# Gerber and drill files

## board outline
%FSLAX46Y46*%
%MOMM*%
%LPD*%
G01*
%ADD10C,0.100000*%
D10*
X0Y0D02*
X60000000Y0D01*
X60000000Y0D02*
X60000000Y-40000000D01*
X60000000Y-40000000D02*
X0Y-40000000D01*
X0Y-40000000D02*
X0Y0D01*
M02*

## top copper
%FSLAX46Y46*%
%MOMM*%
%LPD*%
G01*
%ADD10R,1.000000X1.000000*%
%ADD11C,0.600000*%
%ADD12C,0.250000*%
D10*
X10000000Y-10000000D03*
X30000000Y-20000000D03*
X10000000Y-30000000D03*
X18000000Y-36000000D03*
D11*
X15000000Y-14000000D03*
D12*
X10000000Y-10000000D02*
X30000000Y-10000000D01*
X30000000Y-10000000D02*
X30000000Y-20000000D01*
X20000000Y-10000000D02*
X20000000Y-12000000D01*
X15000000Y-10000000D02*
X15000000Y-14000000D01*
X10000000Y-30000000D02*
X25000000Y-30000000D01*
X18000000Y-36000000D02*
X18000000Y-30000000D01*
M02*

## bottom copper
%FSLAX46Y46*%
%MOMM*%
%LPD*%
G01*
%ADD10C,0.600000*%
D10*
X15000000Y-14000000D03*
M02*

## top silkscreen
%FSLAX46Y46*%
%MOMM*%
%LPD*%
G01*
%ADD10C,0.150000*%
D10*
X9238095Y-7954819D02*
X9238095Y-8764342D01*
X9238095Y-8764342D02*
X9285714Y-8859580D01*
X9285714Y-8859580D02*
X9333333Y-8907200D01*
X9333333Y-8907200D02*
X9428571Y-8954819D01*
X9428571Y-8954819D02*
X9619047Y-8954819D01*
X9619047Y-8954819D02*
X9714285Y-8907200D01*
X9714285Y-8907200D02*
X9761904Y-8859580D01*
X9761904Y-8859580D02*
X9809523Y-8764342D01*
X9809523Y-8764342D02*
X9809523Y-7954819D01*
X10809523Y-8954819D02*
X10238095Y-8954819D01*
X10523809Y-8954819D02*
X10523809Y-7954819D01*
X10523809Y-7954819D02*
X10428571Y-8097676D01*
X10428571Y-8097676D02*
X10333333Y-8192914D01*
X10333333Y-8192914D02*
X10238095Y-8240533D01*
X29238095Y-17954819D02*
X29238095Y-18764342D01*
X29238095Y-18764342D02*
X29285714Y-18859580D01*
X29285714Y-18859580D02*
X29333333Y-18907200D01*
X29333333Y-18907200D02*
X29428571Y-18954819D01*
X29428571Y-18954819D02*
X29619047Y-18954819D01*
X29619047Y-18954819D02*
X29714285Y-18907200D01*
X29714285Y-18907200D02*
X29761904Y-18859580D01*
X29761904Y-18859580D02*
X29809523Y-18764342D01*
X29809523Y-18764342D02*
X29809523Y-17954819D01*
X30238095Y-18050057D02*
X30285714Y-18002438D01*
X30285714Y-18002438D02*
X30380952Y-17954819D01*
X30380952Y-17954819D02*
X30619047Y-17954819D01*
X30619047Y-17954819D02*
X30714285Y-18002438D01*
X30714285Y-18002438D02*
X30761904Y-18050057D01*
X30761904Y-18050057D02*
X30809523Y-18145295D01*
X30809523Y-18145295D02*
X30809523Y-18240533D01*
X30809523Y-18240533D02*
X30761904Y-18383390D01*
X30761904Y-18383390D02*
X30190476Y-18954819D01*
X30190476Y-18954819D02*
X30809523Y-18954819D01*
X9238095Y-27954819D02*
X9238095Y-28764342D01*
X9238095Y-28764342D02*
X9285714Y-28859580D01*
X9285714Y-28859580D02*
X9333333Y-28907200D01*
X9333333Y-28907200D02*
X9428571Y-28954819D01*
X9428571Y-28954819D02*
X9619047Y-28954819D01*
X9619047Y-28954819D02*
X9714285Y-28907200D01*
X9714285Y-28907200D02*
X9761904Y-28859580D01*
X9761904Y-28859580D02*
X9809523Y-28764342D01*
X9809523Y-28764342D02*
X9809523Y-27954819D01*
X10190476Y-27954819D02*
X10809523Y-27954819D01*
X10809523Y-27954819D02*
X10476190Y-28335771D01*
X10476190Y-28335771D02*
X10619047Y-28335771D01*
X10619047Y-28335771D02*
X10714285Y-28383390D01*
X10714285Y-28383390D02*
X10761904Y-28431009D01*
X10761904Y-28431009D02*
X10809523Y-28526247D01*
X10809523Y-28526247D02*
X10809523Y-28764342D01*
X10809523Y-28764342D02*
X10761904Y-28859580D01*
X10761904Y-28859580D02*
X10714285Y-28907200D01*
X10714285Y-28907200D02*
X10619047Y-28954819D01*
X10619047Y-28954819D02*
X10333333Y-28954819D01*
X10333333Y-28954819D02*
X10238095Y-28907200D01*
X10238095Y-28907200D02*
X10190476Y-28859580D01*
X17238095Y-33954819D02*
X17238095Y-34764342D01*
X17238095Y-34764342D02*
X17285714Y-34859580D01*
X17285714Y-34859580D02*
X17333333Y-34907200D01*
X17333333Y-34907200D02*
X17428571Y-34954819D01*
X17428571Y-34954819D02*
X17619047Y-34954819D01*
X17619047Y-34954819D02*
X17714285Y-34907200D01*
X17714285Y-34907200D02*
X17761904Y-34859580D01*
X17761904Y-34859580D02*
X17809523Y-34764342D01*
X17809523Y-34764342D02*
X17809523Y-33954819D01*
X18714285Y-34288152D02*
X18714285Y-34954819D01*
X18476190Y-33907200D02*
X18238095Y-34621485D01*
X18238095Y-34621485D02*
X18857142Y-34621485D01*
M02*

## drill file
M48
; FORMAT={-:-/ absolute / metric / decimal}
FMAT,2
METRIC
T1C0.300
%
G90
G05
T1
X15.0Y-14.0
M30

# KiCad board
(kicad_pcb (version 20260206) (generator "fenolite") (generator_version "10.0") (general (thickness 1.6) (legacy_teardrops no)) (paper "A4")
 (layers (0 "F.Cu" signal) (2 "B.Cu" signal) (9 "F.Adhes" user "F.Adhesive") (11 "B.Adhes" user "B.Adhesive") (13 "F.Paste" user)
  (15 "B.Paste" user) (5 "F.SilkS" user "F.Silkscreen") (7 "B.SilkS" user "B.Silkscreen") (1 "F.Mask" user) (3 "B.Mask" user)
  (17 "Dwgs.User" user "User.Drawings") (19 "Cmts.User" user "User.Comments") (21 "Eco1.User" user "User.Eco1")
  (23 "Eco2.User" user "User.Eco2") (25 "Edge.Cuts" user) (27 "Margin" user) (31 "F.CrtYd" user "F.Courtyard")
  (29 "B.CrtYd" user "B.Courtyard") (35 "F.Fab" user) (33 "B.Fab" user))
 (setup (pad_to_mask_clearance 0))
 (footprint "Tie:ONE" (layer "F.Cu") (at 10 10)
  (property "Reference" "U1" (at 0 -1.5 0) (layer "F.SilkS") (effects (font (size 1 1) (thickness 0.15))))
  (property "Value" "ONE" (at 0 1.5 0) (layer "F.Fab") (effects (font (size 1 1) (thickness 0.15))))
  (pad "1" smd rect (at 0 0) (size 1 1) (layers "F.Cu" "F.Paste" "F.Mask") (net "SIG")))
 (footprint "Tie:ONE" (layer "F.Cu") (at 30 20)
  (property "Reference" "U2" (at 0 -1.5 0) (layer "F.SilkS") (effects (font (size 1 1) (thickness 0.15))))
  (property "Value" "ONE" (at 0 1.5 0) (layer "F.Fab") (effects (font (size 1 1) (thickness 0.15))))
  (pad "1" smd rect (at 0 0) (size 1 1) (layers "F.Cu" "F.Paste" "F.Mask") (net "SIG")))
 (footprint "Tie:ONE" (layer "F.Cu") (at 10 30)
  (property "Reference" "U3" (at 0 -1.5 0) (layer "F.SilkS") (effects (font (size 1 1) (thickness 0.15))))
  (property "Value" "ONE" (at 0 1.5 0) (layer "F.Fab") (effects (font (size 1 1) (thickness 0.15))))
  (pad "1" smd rect (at 0 0) (size 1 1) (layers "F.Cu" "F.Paste" "F.Mask") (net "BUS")))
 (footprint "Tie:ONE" (layer "F.Cu") (at 18 36)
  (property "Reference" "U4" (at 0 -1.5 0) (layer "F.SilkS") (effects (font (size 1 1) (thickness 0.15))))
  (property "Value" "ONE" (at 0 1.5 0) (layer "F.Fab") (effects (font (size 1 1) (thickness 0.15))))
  (pad "1" smd rect (at 0 0) (size 1 1) (layers "F.Cu" "F.Paste" "F.Mask") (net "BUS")))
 (gr_line (start 0 0) (end 60 0) (stroke (width 0.1) (type solid)) (layer "Edge.Cuts"))
 (gr_line (start 60 0) (end 60 40) (stroke (width 0.1) (type solid)) (layer "Edge.Cuts"))
 (gr_line (start 60 40) (end 0 40) (stroke (width 0.1) (type solid)) (layer "Edge.Cuts"))
 (gr_line (start 0 40) (end 0 0) (stroke (width 0.1) (type solid)) (layer "Edge.Cuts"))
 (segment (start 10 10) (end 30 10) (width 0.25) (layer "F.Cu") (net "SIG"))
 (segment (start 30 10) (end 30 20) (width 0.25) (layer "F.Cu") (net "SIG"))
 (segment (start 20 10) (end 20 12) (width 0.25) (layer "F.Cu") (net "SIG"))
 (segment (start 15 10) (end 15 14) (width 0.25) (layer "F.Cu") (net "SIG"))
 (segment (start 10 30) (end 25 30) (width 0.25) (layer "F.Cu") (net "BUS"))
 (segment (start 18 36) (end 18 30) (width 0.25) (layer "F.Cu") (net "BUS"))
 (via (at 15 14) (size 0.6) (drill 0.3) (layers "F.Cu" "B.Cu") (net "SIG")))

